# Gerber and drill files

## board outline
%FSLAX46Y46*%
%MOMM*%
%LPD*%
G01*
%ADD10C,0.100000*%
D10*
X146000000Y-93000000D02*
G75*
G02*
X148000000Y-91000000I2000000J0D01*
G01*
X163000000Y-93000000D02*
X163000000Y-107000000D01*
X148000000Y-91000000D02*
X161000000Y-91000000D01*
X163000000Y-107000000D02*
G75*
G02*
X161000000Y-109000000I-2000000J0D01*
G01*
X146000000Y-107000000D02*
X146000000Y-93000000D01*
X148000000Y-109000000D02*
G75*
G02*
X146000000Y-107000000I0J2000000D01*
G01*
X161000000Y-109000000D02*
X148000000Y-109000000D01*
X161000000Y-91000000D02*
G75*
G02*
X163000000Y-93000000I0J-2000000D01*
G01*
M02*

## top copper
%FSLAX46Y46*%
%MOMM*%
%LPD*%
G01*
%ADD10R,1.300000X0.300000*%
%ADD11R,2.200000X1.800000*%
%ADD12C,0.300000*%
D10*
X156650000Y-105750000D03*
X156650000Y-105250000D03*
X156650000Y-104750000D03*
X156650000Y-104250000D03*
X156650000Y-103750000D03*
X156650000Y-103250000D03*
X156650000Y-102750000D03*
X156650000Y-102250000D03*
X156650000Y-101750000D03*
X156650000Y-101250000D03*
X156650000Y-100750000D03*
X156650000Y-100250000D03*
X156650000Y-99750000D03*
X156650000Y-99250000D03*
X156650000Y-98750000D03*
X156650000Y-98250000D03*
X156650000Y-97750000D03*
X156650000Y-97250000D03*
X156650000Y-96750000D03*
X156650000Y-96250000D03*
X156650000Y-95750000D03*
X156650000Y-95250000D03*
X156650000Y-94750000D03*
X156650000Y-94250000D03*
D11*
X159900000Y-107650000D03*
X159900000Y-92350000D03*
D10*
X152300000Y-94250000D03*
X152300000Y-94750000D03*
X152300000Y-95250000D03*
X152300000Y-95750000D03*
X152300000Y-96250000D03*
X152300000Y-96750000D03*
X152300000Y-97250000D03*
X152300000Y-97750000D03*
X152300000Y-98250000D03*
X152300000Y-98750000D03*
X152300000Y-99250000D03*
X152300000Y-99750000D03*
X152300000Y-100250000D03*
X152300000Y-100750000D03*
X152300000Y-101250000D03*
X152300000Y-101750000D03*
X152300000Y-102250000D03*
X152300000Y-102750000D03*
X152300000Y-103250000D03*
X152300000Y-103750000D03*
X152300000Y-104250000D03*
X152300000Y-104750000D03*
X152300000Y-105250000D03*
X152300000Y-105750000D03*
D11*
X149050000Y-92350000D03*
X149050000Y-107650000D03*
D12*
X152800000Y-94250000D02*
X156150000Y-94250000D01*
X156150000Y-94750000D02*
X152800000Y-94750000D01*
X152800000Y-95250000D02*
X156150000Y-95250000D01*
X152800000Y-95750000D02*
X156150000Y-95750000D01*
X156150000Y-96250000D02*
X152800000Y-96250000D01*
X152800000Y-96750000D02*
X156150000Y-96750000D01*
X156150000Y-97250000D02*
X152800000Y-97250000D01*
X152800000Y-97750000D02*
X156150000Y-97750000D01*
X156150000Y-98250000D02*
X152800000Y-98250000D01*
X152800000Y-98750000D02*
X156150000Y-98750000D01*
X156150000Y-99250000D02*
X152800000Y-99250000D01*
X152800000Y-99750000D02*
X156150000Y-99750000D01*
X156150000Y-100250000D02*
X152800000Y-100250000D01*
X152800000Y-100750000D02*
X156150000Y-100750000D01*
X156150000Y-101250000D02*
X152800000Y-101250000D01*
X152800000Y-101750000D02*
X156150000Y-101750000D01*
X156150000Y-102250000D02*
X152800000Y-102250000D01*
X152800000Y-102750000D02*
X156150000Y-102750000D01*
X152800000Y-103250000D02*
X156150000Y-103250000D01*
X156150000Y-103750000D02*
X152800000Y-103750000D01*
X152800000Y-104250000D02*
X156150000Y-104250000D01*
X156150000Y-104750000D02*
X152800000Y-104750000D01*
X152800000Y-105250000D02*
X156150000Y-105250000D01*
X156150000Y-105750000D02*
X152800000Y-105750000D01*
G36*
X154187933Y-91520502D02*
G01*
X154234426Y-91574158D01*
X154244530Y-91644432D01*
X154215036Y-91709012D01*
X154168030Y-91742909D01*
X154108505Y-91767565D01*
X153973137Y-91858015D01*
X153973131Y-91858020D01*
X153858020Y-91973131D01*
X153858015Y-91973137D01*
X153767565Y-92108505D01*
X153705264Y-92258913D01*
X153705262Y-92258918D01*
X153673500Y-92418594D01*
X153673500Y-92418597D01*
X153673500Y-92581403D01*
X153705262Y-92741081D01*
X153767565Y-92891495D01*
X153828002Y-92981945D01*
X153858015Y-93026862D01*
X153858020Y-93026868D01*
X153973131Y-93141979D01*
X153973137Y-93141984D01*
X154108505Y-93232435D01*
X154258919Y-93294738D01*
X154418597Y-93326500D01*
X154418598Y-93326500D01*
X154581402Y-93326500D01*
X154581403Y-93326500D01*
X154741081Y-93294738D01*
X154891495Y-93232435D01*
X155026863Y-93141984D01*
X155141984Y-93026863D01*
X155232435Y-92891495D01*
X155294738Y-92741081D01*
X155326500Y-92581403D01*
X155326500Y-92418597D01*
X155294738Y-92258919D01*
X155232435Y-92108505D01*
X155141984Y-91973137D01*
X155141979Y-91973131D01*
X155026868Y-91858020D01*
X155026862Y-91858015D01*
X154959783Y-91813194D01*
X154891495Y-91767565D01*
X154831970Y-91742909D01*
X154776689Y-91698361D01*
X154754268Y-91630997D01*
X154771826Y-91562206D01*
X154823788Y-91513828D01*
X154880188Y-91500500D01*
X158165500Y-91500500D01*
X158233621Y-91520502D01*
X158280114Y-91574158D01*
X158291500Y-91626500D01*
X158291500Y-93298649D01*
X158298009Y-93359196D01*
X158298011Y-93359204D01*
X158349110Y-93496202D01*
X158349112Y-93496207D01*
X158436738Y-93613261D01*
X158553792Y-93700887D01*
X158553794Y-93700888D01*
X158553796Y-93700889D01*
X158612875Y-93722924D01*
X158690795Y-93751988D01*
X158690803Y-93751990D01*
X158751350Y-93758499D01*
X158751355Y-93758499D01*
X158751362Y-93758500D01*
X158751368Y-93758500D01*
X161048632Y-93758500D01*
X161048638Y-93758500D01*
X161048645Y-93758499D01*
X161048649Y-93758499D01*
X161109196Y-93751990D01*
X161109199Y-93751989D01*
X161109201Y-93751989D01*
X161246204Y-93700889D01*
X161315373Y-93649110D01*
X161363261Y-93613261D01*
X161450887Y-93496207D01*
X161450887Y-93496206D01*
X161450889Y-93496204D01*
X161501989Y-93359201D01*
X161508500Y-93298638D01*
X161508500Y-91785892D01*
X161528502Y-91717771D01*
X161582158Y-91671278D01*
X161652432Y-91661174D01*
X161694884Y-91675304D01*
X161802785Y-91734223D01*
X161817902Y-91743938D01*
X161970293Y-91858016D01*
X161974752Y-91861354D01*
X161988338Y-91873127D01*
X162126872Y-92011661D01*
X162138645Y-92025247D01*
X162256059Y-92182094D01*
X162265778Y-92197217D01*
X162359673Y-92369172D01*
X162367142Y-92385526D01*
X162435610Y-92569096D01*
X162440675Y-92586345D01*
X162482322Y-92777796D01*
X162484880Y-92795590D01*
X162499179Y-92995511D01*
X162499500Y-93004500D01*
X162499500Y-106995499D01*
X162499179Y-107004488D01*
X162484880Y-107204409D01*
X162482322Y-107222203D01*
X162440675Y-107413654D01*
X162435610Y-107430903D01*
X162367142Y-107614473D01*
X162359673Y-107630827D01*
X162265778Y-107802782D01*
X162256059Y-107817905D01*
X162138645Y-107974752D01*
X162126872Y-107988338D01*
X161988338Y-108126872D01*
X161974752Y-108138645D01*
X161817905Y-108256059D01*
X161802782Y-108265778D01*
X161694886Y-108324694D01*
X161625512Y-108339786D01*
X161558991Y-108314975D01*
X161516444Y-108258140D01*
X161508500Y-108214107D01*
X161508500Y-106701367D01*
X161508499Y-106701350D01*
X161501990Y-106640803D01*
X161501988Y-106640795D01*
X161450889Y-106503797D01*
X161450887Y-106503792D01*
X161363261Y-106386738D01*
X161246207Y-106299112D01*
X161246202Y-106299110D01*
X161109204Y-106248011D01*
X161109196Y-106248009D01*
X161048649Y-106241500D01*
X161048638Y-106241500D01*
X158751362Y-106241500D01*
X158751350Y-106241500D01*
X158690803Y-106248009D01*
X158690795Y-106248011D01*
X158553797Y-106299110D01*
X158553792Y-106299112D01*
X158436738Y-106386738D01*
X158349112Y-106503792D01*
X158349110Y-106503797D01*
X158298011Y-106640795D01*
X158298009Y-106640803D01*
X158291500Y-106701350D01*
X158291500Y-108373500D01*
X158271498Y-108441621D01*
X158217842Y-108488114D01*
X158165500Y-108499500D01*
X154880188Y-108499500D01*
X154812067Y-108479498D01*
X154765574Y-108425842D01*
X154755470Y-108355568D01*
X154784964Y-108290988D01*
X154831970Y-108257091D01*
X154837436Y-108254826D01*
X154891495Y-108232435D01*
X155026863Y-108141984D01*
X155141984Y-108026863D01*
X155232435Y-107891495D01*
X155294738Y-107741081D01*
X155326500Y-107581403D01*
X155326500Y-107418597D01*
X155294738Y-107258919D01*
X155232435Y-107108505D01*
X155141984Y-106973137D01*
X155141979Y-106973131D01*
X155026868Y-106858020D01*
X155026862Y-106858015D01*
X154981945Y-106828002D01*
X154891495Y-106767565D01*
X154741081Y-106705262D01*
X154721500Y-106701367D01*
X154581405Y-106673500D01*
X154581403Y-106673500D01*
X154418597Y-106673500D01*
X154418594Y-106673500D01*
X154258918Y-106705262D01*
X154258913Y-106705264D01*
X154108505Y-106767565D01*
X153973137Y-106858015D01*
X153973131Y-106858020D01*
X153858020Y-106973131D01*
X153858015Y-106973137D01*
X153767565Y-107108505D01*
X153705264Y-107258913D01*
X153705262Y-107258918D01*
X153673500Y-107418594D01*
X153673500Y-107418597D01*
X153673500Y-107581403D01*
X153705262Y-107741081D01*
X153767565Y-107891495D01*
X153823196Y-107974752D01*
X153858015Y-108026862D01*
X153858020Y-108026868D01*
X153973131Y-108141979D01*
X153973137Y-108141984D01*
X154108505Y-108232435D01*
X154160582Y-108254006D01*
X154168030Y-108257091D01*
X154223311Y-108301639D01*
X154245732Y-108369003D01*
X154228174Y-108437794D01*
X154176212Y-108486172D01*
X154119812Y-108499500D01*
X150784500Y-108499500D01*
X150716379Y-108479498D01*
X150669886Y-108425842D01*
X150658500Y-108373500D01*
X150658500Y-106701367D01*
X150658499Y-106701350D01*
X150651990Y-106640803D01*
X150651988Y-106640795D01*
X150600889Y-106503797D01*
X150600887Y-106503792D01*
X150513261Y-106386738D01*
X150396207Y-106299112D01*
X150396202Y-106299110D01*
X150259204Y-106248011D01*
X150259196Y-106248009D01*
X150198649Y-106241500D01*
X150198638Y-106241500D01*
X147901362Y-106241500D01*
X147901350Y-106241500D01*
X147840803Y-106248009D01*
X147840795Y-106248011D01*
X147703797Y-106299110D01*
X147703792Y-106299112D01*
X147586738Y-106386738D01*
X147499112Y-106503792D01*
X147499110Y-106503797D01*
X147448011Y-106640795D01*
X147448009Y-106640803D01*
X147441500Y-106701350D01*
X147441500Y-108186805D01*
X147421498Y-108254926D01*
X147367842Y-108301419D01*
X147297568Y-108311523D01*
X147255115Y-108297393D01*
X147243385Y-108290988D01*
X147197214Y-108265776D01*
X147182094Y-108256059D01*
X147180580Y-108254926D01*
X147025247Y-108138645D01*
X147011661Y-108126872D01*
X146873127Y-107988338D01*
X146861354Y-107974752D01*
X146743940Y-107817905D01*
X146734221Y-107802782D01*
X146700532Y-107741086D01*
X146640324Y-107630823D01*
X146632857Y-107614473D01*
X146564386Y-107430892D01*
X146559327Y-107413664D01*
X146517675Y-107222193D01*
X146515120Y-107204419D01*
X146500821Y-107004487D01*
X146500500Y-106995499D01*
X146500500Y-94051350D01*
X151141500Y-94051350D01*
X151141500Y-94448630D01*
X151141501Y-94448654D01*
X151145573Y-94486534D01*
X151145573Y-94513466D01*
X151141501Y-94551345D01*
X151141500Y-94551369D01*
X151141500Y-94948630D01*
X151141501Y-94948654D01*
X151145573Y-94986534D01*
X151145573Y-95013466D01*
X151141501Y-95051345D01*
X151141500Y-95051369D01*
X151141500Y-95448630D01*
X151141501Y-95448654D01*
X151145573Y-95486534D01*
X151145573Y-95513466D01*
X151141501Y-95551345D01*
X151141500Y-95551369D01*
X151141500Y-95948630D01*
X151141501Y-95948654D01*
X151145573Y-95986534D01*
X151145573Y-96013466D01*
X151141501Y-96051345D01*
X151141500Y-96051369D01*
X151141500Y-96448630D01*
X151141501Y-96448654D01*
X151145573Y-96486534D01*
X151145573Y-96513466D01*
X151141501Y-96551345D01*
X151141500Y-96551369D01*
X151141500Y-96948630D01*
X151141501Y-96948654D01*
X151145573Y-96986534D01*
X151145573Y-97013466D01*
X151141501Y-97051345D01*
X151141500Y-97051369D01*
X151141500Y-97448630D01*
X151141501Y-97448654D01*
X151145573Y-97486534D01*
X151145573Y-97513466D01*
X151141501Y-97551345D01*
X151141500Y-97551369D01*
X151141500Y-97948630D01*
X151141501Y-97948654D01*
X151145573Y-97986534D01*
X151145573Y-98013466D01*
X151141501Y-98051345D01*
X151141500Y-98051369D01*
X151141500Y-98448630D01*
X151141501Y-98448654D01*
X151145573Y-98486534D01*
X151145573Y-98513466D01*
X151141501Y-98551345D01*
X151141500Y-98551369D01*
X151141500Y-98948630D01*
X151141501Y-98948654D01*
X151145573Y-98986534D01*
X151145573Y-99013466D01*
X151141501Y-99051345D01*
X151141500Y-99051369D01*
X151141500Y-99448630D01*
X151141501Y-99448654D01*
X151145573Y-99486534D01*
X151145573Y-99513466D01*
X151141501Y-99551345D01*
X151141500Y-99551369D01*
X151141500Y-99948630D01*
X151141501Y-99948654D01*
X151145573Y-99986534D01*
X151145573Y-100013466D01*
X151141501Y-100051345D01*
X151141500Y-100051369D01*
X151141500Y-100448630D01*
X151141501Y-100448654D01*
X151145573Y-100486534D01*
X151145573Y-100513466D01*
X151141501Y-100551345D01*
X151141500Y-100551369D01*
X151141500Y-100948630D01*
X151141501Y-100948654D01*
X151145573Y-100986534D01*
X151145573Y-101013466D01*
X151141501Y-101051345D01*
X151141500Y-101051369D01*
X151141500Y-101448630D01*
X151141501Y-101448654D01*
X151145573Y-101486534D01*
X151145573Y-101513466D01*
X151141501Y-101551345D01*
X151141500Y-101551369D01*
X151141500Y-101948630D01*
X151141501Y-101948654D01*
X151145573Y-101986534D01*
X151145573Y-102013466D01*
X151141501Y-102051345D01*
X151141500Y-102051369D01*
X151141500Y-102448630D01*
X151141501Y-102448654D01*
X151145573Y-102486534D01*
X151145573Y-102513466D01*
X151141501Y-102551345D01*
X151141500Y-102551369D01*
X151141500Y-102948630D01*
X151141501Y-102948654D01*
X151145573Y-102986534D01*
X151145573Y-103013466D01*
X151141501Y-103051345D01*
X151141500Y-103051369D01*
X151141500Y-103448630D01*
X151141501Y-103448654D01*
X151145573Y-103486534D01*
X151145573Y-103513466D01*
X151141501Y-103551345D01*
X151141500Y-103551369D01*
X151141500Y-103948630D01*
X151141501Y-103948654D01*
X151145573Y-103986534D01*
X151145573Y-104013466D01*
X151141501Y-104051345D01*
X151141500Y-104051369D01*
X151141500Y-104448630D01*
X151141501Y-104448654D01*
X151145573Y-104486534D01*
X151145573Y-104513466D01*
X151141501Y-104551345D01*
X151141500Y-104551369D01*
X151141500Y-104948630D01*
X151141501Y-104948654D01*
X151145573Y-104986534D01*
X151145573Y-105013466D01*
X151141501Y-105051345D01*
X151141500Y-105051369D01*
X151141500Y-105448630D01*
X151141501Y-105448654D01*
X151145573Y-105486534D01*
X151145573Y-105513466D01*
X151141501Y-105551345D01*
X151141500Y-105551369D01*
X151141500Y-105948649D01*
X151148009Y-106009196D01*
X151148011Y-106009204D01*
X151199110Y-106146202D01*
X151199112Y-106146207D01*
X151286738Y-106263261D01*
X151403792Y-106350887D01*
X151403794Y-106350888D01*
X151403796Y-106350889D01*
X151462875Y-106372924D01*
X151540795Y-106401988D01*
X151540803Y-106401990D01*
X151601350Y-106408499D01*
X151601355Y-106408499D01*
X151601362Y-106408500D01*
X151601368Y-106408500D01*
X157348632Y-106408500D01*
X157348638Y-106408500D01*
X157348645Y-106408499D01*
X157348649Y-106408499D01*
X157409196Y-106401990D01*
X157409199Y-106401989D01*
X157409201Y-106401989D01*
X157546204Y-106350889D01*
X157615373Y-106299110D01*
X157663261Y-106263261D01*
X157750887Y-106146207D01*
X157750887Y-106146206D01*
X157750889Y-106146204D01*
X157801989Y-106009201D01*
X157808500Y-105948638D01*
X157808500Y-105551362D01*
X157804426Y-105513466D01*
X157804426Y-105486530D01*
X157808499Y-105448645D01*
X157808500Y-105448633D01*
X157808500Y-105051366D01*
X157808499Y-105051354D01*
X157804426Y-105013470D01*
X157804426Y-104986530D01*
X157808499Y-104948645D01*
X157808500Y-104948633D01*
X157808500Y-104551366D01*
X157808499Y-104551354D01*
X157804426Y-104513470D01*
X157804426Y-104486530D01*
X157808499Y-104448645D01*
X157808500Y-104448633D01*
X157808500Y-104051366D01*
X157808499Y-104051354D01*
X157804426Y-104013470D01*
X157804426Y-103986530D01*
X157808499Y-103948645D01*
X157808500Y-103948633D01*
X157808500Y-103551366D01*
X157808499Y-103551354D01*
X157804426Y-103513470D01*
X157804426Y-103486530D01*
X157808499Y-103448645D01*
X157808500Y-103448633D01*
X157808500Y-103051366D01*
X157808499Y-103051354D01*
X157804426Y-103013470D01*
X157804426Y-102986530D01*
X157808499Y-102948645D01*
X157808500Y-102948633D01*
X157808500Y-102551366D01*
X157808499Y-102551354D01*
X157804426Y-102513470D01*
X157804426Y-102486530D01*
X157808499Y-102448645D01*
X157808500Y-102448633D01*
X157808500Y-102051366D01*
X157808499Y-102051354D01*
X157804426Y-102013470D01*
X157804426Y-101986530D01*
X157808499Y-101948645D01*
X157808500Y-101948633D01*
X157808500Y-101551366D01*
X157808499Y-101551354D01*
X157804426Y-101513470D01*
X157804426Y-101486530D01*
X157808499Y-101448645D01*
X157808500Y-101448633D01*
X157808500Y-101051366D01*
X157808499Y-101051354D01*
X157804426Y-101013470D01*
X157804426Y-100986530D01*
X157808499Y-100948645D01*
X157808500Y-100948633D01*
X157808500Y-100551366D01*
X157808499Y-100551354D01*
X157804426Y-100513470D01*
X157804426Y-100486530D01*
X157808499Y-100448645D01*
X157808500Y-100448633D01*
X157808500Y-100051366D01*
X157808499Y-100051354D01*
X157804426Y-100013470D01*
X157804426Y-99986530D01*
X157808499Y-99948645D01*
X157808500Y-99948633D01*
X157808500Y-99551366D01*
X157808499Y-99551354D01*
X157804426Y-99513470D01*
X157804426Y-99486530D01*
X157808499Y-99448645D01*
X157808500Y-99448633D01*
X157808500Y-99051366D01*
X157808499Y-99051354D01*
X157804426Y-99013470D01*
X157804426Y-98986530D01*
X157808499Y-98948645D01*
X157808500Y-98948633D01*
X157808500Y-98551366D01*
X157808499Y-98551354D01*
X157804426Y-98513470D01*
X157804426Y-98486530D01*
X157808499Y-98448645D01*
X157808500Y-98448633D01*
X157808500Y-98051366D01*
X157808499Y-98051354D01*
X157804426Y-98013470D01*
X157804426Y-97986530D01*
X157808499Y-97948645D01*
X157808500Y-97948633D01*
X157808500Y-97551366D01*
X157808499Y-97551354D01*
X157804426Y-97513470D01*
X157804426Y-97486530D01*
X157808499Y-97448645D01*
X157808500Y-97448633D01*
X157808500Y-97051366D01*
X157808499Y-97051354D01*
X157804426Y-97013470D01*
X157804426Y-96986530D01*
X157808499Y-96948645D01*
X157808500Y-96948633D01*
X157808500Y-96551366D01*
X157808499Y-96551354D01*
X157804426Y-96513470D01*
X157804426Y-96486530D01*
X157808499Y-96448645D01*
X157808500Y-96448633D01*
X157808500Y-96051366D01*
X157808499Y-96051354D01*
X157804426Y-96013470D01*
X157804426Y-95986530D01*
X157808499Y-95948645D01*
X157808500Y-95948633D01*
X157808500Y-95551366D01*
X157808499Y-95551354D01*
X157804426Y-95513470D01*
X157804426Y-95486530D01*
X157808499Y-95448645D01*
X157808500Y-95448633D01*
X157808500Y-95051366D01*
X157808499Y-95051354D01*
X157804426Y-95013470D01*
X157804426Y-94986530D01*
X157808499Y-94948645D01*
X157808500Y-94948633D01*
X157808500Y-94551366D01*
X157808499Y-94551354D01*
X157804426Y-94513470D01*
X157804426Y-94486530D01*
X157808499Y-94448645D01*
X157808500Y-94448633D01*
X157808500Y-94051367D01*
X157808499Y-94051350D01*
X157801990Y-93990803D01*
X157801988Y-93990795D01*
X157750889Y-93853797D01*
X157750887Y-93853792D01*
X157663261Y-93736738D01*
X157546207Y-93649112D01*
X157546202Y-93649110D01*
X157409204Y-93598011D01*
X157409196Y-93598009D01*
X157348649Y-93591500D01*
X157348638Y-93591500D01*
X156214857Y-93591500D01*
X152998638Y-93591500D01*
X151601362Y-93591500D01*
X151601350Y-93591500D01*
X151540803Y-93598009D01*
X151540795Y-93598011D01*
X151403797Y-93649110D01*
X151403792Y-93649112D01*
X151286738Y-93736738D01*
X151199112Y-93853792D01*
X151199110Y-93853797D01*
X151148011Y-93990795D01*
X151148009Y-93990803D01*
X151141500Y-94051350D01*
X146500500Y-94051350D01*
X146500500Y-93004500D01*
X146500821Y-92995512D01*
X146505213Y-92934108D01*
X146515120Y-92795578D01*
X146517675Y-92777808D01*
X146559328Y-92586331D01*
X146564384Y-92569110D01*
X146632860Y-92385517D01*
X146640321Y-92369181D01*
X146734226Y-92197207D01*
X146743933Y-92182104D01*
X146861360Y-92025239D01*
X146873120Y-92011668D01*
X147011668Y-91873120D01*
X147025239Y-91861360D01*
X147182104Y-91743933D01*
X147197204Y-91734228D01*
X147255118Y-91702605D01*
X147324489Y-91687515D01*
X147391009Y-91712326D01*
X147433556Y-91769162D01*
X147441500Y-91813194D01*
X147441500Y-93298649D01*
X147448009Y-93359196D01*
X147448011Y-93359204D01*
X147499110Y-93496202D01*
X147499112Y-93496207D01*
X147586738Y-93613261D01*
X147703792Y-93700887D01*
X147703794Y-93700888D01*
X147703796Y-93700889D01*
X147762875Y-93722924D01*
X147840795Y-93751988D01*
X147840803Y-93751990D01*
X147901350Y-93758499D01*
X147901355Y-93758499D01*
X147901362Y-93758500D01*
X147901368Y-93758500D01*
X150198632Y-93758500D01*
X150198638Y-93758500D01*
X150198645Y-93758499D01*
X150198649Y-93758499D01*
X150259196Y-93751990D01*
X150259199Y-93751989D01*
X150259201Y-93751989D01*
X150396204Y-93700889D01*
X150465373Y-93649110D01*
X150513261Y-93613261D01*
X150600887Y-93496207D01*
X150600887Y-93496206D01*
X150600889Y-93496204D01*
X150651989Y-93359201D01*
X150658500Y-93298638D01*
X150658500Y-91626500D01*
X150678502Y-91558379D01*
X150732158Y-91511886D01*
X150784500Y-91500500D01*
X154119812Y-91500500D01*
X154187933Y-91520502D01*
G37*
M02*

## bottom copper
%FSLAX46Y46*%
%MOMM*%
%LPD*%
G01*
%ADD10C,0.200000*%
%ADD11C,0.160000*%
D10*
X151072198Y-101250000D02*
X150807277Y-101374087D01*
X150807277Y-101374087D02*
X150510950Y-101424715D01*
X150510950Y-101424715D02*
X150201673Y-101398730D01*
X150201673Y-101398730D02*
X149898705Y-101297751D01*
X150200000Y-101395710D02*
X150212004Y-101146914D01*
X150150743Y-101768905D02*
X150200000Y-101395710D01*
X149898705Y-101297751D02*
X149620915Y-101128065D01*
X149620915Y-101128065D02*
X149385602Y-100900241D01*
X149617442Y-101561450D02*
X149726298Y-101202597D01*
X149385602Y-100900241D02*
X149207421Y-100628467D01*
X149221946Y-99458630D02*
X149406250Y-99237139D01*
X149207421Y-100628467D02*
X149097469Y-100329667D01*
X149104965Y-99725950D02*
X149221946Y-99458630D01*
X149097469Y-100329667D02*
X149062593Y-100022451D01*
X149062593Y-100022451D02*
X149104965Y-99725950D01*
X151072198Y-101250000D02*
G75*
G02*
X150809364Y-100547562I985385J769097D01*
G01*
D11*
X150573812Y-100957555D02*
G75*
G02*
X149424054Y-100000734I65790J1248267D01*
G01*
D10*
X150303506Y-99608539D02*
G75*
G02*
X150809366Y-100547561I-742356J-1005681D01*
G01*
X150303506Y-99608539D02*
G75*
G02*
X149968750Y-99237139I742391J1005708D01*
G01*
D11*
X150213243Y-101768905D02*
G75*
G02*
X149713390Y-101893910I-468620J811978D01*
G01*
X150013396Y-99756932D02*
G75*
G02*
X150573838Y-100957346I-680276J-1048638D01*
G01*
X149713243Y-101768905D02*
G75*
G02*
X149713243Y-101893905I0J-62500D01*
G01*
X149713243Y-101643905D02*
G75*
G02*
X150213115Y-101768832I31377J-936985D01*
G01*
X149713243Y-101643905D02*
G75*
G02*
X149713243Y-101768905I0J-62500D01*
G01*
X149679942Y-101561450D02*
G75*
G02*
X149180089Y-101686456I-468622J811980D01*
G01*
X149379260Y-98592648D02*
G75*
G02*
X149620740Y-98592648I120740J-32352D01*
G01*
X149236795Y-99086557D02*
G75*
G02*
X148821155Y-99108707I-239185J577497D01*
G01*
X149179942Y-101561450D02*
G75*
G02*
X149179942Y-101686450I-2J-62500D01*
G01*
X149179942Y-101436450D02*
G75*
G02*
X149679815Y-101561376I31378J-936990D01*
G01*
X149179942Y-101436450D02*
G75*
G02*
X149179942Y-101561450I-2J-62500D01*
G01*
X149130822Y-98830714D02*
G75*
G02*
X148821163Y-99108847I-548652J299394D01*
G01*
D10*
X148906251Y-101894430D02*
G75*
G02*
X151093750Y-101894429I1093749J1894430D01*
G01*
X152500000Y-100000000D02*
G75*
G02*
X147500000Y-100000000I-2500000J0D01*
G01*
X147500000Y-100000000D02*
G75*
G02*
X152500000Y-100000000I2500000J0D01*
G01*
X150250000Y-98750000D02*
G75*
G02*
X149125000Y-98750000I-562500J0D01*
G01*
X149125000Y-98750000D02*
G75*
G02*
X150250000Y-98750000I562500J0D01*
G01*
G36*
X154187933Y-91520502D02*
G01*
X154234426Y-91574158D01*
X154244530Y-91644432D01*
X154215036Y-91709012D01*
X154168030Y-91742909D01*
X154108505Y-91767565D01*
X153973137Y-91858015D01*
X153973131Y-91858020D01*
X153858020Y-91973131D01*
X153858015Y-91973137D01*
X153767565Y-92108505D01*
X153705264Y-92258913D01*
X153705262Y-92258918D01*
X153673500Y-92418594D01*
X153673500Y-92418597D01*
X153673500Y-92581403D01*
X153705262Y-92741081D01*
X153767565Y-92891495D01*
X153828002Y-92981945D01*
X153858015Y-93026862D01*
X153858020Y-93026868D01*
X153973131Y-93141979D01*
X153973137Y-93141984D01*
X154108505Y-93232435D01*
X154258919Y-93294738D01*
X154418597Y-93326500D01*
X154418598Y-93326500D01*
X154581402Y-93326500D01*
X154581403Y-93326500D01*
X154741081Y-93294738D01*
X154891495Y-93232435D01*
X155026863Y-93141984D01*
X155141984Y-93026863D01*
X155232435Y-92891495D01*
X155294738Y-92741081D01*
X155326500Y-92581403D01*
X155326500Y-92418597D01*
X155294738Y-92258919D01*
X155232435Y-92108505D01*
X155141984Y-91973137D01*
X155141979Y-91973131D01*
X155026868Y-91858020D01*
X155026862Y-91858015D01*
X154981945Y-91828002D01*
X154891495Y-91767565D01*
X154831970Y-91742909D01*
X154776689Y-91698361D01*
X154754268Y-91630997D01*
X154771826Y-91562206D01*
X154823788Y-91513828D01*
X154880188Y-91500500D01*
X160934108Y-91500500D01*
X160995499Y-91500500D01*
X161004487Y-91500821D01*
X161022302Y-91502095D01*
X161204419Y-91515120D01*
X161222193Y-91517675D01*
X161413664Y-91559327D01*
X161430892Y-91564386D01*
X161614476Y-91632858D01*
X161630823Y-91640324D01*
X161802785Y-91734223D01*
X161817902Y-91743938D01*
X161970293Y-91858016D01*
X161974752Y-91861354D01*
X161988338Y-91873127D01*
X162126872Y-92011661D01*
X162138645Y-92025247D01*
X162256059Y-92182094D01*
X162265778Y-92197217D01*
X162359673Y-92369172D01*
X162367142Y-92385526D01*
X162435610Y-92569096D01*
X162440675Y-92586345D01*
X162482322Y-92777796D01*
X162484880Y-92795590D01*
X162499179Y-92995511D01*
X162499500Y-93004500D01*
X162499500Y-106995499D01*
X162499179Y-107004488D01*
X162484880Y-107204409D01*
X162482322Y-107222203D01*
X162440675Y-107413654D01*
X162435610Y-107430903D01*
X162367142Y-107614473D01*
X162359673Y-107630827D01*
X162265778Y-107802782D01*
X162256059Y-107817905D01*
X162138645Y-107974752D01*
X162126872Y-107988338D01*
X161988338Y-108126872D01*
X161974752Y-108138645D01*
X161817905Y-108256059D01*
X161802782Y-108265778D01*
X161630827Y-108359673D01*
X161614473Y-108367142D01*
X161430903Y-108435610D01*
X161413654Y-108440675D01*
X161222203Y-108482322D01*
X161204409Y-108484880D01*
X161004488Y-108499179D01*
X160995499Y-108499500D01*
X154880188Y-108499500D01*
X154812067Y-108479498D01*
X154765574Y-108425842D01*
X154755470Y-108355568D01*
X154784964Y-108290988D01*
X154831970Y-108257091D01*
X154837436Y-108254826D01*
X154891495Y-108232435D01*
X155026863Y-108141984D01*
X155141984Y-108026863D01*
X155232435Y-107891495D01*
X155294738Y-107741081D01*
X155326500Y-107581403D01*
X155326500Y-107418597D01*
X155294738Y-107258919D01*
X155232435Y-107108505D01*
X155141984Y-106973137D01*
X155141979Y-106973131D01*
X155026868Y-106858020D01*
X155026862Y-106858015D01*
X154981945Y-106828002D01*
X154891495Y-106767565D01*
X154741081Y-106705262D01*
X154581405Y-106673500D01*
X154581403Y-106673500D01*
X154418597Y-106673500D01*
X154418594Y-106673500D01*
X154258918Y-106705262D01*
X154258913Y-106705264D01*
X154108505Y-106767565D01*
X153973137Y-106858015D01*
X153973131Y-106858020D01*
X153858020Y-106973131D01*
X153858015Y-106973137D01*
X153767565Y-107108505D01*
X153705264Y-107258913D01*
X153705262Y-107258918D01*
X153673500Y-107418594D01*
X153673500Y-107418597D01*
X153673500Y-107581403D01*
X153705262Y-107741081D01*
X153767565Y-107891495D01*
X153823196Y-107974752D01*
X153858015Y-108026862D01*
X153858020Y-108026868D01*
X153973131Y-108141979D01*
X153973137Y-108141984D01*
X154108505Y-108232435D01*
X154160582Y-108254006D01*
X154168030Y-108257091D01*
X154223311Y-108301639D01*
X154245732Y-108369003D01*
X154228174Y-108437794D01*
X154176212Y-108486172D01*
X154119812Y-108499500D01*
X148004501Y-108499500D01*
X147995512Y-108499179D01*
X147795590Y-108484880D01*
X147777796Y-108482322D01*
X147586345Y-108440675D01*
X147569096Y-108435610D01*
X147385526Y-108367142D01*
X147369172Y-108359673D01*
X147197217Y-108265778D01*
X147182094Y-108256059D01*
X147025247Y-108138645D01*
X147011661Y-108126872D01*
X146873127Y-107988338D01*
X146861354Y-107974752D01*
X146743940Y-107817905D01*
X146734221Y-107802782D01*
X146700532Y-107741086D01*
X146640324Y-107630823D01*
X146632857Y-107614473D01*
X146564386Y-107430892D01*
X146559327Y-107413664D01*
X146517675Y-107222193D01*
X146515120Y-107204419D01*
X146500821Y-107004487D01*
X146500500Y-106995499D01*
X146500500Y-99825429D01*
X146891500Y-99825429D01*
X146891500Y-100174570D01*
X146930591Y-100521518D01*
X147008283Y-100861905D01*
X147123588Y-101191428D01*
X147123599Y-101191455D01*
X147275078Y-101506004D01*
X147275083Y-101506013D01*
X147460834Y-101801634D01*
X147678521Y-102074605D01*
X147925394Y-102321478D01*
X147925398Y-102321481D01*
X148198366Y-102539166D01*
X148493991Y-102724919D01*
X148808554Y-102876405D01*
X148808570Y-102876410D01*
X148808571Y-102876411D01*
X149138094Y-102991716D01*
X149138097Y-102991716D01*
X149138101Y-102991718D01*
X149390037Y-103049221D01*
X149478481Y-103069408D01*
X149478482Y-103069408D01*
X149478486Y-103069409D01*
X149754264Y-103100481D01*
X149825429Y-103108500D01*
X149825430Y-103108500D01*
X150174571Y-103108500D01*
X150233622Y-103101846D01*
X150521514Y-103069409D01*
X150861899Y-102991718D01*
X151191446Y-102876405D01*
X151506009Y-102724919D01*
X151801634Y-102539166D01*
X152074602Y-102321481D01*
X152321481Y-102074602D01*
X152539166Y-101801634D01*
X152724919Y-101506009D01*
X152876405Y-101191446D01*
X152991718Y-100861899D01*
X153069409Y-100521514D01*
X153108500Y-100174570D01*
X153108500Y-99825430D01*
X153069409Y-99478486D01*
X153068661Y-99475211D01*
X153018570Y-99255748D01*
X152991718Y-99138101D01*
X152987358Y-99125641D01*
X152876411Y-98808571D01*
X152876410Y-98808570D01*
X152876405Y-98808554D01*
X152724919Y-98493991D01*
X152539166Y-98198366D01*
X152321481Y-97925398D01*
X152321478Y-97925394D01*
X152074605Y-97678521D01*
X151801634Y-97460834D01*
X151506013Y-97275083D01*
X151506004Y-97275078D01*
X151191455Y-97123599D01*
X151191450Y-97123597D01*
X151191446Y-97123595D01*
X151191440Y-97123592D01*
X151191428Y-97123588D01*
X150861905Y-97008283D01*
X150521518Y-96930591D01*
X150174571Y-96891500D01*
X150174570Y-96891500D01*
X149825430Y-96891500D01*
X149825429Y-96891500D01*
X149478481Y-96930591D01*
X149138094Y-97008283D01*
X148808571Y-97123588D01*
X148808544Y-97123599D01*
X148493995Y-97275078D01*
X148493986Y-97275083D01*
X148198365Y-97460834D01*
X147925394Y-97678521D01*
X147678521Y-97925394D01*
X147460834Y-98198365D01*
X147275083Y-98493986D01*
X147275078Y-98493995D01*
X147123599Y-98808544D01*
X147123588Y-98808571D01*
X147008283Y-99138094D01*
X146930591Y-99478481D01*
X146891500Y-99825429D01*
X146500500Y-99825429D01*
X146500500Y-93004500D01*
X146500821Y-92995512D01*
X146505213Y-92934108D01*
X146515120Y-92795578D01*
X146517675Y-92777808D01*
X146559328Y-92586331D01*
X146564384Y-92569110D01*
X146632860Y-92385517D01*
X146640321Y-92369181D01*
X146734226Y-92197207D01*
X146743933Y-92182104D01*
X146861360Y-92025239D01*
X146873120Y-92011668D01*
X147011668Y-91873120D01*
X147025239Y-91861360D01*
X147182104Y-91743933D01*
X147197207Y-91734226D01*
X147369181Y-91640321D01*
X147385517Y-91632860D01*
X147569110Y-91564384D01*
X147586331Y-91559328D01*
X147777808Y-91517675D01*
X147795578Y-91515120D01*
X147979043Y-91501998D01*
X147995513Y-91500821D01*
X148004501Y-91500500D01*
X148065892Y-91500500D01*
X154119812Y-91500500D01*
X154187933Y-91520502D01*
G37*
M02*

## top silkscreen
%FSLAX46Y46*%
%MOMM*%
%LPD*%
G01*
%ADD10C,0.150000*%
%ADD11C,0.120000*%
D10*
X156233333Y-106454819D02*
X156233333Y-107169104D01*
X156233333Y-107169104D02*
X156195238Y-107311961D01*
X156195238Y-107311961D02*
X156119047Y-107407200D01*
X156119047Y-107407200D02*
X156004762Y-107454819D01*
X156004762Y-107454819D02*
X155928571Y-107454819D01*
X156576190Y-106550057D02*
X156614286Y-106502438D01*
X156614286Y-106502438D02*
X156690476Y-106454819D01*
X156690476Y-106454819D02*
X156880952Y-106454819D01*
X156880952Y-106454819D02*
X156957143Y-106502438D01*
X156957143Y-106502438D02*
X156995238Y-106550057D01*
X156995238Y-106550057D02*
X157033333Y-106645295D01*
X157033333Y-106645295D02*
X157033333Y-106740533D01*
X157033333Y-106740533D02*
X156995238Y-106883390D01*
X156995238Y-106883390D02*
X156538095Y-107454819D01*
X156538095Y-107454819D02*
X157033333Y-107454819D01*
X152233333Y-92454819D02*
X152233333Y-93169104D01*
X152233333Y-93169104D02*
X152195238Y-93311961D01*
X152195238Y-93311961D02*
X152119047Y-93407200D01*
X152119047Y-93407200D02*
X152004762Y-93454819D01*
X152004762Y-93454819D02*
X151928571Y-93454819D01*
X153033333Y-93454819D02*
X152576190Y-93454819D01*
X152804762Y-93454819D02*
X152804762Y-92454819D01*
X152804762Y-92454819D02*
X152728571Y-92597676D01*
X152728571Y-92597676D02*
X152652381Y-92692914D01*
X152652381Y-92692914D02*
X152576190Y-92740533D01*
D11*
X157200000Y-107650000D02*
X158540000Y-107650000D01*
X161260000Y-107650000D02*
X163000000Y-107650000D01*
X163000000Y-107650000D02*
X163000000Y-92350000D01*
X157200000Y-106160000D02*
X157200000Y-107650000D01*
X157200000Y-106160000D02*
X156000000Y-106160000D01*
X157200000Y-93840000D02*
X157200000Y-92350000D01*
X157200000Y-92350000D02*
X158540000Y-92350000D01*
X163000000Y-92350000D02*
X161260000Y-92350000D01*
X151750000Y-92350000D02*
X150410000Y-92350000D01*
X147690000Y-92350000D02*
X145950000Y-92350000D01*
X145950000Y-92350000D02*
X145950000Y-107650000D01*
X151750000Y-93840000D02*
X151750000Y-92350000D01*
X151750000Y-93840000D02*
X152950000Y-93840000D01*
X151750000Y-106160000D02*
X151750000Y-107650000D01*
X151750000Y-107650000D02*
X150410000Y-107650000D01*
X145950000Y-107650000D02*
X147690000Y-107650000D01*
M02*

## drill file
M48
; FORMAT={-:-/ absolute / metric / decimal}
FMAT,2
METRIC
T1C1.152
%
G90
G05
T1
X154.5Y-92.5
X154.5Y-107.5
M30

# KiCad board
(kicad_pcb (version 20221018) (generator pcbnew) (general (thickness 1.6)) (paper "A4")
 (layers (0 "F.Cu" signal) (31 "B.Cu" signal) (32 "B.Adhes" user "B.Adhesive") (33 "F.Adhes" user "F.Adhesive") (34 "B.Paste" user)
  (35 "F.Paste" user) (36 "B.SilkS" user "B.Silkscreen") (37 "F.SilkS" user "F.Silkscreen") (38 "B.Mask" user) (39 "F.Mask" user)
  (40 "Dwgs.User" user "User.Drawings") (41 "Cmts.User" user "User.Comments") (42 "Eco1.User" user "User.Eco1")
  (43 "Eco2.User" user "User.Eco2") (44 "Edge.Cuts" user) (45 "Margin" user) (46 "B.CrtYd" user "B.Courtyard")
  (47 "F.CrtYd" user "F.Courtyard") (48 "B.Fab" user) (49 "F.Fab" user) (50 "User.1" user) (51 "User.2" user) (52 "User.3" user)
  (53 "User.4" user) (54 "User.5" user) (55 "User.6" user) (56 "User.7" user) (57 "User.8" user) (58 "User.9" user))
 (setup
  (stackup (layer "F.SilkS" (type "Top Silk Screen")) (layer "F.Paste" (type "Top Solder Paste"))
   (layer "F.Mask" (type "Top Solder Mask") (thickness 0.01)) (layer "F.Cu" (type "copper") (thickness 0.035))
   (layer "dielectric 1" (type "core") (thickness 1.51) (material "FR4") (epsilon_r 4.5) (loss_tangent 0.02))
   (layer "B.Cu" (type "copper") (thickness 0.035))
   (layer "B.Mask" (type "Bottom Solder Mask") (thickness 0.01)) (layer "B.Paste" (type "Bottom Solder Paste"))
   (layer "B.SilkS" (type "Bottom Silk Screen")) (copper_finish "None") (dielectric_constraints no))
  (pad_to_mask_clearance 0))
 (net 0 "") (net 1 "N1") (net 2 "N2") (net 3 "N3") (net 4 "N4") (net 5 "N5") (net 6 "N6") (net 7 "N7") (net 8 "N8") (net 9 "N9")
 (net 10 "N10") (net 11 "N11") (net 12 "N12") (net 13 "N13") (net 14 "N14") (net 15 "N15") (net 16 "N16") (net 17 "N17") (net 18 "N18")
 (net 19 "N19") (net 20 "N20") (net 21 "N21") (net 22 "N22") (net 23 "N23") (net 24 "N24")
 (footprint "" (layer "F.Cu") (at 154.5 92.5)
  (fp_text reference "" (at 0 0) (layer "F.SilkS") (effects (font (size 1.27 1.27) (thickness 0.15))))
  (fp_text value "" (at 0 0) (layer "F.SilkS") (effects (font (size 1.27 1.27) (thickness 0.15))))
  (pad "" np_thru_hole circle (at 0 0) (size 1.152 1.152) (drill 1.152) (layers "F&B.Cu" "*.Mask")))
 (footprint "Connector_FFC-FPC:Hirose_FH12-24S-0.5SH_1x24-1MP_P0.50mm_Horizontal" (layer "F.Cu") (at 158.5 100 90)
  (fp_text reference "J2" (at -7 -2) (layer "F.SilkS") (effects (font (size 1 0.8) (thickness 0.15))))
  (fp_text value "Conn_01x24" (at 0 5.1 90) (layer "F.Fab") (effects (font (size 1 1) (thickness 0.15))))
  (fp_line (start -7.65 -1.3) (end -7.65 0.04) (stroke (width 0.12) (type solid)) (layer "F.SilkS"))
  (fp_line (start -7.65 2.76) (end -7.65 4.5) (stroke (width 0.12) (type solid)) (layer "F.SilkS"))
  (fp_line (start -7.65 4.5) (end 7.65 4.5) (stroke (width 0.12) (type solid)) (layer "F.SilkS"))
  (fp_line (start -6.16 -1.3) (end -7.65 -1.3) (stroke (width 0.12) (type solid)) (layer "F.SilkS"))
  (fp_line (start -6.16 -1.3) (end -6.16 -2.5) (stroke (width 0.12) (type solid)) (layer "F.SilkS"))
  (fp_line (start 6.16 -1.3) (end 7.65 -1.3) (stroke (width 0.12) (type solid)) (layer "F.SilkS"))
  (fp_line (start 7.65 -1.3) (end 7.65 0.04) (stroke (width 0.12) (type solid)) (layer "F.SilkS"))
  (fp_line (start 7.65 4.5) (end 7.65 2.76) (stroke (width 0.12) (type solid)) (layer "F.SilkS"))
  (pad "1" smd rect (at -5.75 -1.85 90) (size 0.3 1.3) (layers "F.Cu" "F.Paste" "F.Mask") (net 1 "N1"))
  (pad "2" smd rect (at -5.25 -1.85 90) (size 0.3 1.3) (layers "F.Cu" "F.Paste" "F.Mask") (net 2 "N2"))
  (pad "3" smd rect (at -4.75 -1.85 90) (size 0.3 1.3) (layers "F.Cu" "F.Paste" "F.Mask") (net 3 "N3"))
  (pad "4" smd rect (at -4.25 -1.85 90) (size 0.3 1.3) (layers "F.Cu" "F.Paste" "F.Mask") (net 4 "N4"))
  (pad "5" smd rect (at -3.75 -1.85 90) (size 0.3 1.3) (layers "F.Cu" "F.Paste" "F.Mask") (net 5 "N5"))
  (pad "6" smd rect (at -3.25 -1.85 90) (size 0.3 1.3) (layers "F.Cu" "F.Paste" "F.Mask") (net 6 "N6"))
  (pad "7" smd rect (at -2.75 -1.85 90) (size 0.3 1.3) (layers "F.Cu" "F.Paste" "F.Mask") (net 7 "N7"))
  (pad "8" smd rect (at -2.25 -1.85 90) (size 0.3 1.3) (layers "F.Cu" "F.Paste" "F.Mask") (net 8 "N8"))
  (pad "9" smd rect (at -1.75 -1.85 90) (size 0.3 1.3) (layers "F.Cu" "F.Paste" "F.Mask") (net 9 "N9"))
  (pad "10" smd rect (at -1.25 -1.85 90) (size 0.3 1.3) (layers "F.Cu" "F.Paste" "F.Mask") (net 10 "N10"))
  (pad "11" smd rect (at -0.75 -1.85 90) (size 0.3 1.3) (layers "F.Cu" "F.Paste" "F.Mask") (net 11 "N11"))
  (pad "12" smd rect (at -0.25 -1.85 90) (size 0.3 1.3) (layers "F.Cu" "F.Paste" "F.Mask") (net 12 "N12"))
  (pad "13" smd rect (at 0.25 -1.85 90) (size 0.3 1.3) (layers "F.Cu" "F.Paste" "F.Mask") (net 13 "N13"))
  (pad "14" smd rect (at 0.75 -1.85 90) (size 0.3 1.3) (layers "F.Cu" "F.Paste" "F.Mask") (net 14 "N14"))
  (pad "15" smd rect (at 1.25 -1.85 90) (size 0.3 1.3) (layers "F.Cu" "F.Paste" "F.Mask") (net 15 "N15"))
  (pad "16" smd rect (at 1.75 -1.85 90) (size 0.3 1.3) (layers "F.Cu" "F.Paste" "F.Mask") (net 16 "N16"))
  (pad "17" smd rect (at 2.25 -1.85 90) (size 0.3 1.3) (layers "F.Cu" "F.Paste" "F.Mask") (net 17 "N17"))
  (pad "18" smd rect (at 2.75 -1.85 90) (size 0.3 1.3) (layers "F.Cu" "F.Paste" "F.Mask") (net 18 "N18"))
  (pad "19" smd rect (at 3.25 -1.85 90) (size 0.3 1.3) (layers "F.Cu" "F.Paste" "F.Mask") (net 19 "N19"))
  (pad "20" smd rect (at 3.75 -1.85 90) (size 0.3 1.3) (layers "F.Cu" "F.Paste" "F.Mask") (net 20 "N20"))
  (pad "21" smd rect (at 4.25 -1.85 90) (size 0.3 1.3) (layers "F.Cu" "F.Paste" "F.Mask") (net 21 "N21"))
  (pad "22" smd rect (at 4.75 -1.85 90) (size 0.3 1.3) (layers "F.Cu" "F.Paste" "F.Mask") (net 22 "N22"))
  (pad "23" smd rect (at 5.25 -1.85 90) (size 0.3 1.3) (layers "F.Cu" "F.Paste" "F.Mask") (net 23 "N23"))
  (pad "24" smd rect (at 5.75 -1.85 90) (size 0.3 1.3) (layers "F.Cu" "F.Paste" "F.Mask") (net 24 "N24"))
  (pad "MP" smd rect (at -7.65 1.4 90) (size 1.8 2.2) (layers "F.Cu" "F.Paste" "F.Mask"))
  (pad "MP" smd rect (at 7.65 1.4 90) (size 1.8 2.2) (layers "F.Cu" "F.Paste" "F.Mask")))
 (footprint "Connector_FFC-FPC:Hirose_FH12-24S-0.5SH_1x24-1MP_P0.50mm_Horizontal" (layer "F.Cu") (at 150.45 100 -90)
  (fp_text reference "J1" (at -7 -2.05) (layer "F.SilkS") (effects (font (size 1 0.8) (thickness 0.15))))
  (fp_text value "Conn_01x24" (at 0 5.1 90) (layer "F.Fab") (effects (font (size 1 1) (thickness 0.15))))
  (fp_line (start -7.65 -1.3) (end -7.65 0.04) (stroke (width 0.12) (type solid)) (layer "F.SilkS"))
  (fp_line (start -7.65 2.76) (end -7.65 4.5) (stroke (width 0.12) (type solid)) (layer "F.SilkS"))
  (fp_line (start -7.65 4.5) (end 7.65 4.5) (stroke (width 0.12) (type solid)) (layer "F.SilkS"))
  (fp_line (start -6.16 -1.3) (end -7.65 -1.3) (stroke (width 0.12) (type solid)) (layer "F.SilkS"))
  (fp_line (start -6.16 -1.3) (end -6.16 -2.5) (stroke (width 0.12) (type solid)) (layer "F.SilkS"))
  (fp_line (start 6.16 -1.3) (end 7.65 -1.3) (stroke (width 0.12) (type solid)) (layer "F.SilkS"))
  (fp_line (start 7.65 -1.3) (end 7.65 0.04) (stroke (width 0.12) (type solid)) (layer "F.SilkS"))
  (fp_line (start 7.65 4.5) (end 7.65 2.76) (stroke (width 0.12) (type solid)) (layer "F.SilkS"))
  (pad "1" smd rect (at -5.75 -1.85 270) (size 0.3 1.3) (layers "F.Cu" "F.Paste" "F.Mask") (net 24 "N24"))
  (pad "2" smd rect (at -5.25 -1.85 270) (size 0.3 1.3) (layers "F.Cu" "F.Paste" "F.Mask") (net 23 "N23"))
  (pad "3" smd rect (at -4.75 -1.85 270) (size 0.3 1.3) (layers "F.Cu" "F.Paste" "F.Mask") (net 22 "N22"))
  (pad "4" smd rect (at -4.25 -1.85 270) (size 0.3 1.3) (layers "F.Cu" "F.Paste" "F.Mask") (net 21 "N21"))
  (pad "5" smd rect (at -3.75 -1.85 270) (size 0.3 1.3) (layers "F.Cu" "F.Paste" "F.Mask") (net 20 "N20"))
  (pad "6" smd rect (at -3.25 -1.85 270) (size 0.3 1.3) (layers "F.Cu" "F.Paste" "F.Mask") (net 19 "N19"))
  (pad "7" smd rect (at -2.75 -1.85 270) (size 0.3 1.3) (layers "F.Cu" "F.Paste" "F.Mask") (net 18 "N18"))
  (pad "8" smd rect (at -2.25 -1.85 270) (size 0.3 1.3) (layers "F.Cu" "F.Paste" "F.Mask") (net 17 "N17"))
  (pad "9" smd rect (at -1.75 -1.85 270) (size 0.3 1.3) (layers "F.Cu" "F.Paste" "F.Mask") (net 16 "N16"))
  (pad "10" smd rect (at -1.25 -1.85 270) (size 0.3 1.3) (layers "F.Cu" "F.Paste" "F.Mask") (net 15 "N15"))
  (pad "11" smd rect (at -0.75 -1.85 270) (size 0.3 1.3) (layers "F.Cu" "F.Paste" "F.Mask") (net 14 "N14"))
  (pad "12" smd rect (at -0.25 -1.85 270) (size 0.3 1.3) (layers "F.Cu" "F.Paste" "F.Mask") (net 13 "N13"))
  (pad "13" smd rect (at 0.25 -1.85 270) (size 0.3 1.3) (layers "F.Cu" "F.Paste" "F.Mask") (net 12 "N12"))
  (pad "14" smd rect (at 0.75 -1.85 270) (size 0.3 1.3) (layers "F.Cu" "F.Paste" "F.Mask") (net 11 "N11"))
  (pad "15" smd rect (at 1.25 -1.85 270) (size 0.3 1.3) (layers "F.Cu" "F.Paste" "F.Mask") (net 10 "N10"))
  (pad "16" smd rect (at 1.75 -1.85 270) (size 0.3 1.3) (layers "F.Cu" "F.Paste" "F.Mask") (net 9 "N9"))
  (pad "17" smd rect (at 2.25 -1.85 270) (size 0.3 1.3) (layers "F.Cu" "F.Paste" "F.Mask") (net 8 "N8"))
  (pad "18" smd rect (at 2.75 -1.85 270) (size 0.3 1.3) (layers "F.Cu" "F.Paste" "F.Mask") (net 7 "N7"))
  (pad "19" smd rect (at 3.25 -1.85 270) (size 0.3 1.3) (layers "F.Cu" "F.Paste" "F.Mask") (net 6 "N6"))
  (pad "20" smd rect (at 3.75 -1.85 270) (size 0.3 1.3) (layers "F.Cu" "F.Paste" "F.Mask") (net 5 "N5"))
  (pad "21" smd rect (at 4.25 -1.85 270) (size 0.3 1.3) (layers "F.Cu" "F.Paste" "F.Mask") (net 4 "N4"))
  (pad "22" smd rect (at 4.75 -1.85 270) (size 0.3 1.3) (layers "F.Cu" "F.Paste" "F.Mask") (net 3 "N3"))
  (pad "23" smd rect (at 5.25 -1.85 270) (size 0.3 1.3) (layers "F.Cu" "F.Paste" "F.Mask") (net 2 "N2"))
  (pad "24" smd rect (at 5.75 -1.85 270) (size 0.3 1.3) (layers "F.Cu" "F.Paste" "F.Mask") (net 1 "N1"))
  (pad "MP" smd rect (at -7.65 1.4 270) (size 1.8 2.2) (layers "F.Cu" "F.Paste" "F.Mask"))
  (pad "MP" smd rect (at 7.65 1.4 270) (size 1.8 2.2) (layers "F.Cu" "F.Paste" "F.Mask")))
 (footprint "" (layer "F.Cu") (at 154.5 107.5)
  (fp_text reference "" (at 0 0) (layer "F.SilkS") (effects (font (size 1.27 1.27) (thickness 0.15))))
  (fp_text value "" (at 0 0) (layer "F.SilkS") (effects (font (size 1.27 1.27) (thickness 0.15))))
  (pad "" np_thru_hole circle (at 0 0) (size 1.152 1.152) (drill 1.152) (layers "F&B.Cu" "*.Mask")))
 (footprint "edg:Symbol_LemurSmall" (layer "B.Cu") (at 160 100 180)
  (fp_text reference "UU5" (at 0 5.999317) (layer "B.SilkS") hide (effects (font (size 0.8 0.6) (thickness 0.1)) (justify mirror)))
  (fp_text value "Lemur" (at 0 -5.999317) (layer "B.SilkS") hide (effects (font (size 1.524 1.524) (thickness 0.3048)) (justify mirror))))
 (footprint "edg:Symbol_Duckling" (layer "B.Cu") (at 150 100 180)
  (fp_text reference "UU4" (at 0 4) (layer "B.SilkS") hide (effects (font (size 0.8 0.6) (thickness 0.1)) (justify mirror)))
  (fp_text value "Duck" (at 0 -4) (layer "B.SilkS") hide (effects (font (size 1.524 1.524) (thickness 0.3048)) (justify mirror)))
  (fp_line (start -1.072198 -1.25) (end -0.807277 -1.374087) (stroke (width 0.2) (type solid)) (layer "B.Cu"))
  (fp_line (start -0.807277 -1.374087) (end -0.51095 -1.424715) (stroke (width 0.2) (type solid)) (layer "B.Cu"))
  (fp_line (start -0.51095 -1.424715) (end -0.201673 -1.39873) (stroke (width 0.2) (type solid)) (layer "B.Cu"))
  (fp_line (start -0.201673 -1.39873) (end 0.101295 -1.297751) (stroke (width 0.2) (type solid)) (layer "B.Cu"))
  (fp_line (start -0.2 -1.39571) (end -0.212004 -1.146914) (stroke (width 0.2) (type solid)) (layer "B.Cu"))
  (fp_line (start -0.150743 -1.768905) (end -0.2 -1.39571) (stroke (width 0.2) (type solid)) (layer "B.Cu"))
  (fp_line (start 0.101295 -1.297751) (end 0.379085 -1.128065) (stroke (width 0.2) (type solid)) (layer "B.Cu"))
  (fp_line (start 0.379085 -1.128065) (end 0.614398 -0.900241) (stroke (width 0.2) (type solid)) (layer "B.Cu"))
  (fp_line (start 0.382558 -1.56145) (end 0.273702 -1.202597) (stroke (width 0.2) (type solid)) (layer "B.Cu"))
  (fp_line (start 0.614398 -0.900241) (end 0.792579 -0.628467) (stroke (width 0.2) (type solid)) (layer "B.Cu"))
  (fp_line (start 0.778054 0.54137) (end 0.59375 0.762861) (stroke (width 0.2) (type solid)) (layer "B.Cu"))
  (fp_line (start 0.792579 -0.628467) (end 0.902531 -0.329667) (stroke (width 0.2) (type solid)) (layer "B.Cu"))
  (fp_line (start 0.895035 0.27405) (end 0.778054 0.54137) (stroke (width 0.2) (type solid)) (layer "B.Cu"))
  (fp_line (start 0.902531 -0.329667) (end 0.937407 -0.022451) (stroke (width 0.2) (type solid)) (layer "B.Cu"))
  (fp_line (start 0.937407 -0.022451) (end 0.895035 0.27405) (stroke (width 0.2) (type solid)) (layer "B.Cu"))
  (fp_arc (start -1.072198 -1.25) (mid -0.886856 -0.918958) (end -0.809364 -0.547562) (stroke (width 0.2) (type solid)) (layer "B.Cu"))
  (fp_arc (start -0.573812 -0.957555) (mid 0.159981 -0.670103) (end 0.575946 -0.000734) (stroke (width 0.16) (type solid)) (layer "B.Cu"))
  (fp_arc (start -0.303506 0.391461) (mid -0.66162 -0.021386) (end -0.809366 -0.547561) (stroke (width 0.2) (type solid)) (layer "B.Cu"))
  (fp_arc (start -0.303506 0.391461) (mid -0.117369 0.560253) (end 0.03125 0.762861) (stroke (width 0.2) (type solid)) (layer "B.Cu"))
  (fp_arc (start -0.213243 -1.768905) (mid 0.027927 -1.866421) (end 0.28661 -1.89391) (stroke (width 0.16) (type solid)) (layer "B.Cu"))
  (fp_arc (start -0.013396 0.243068) (mid -0.465729 -0.276784) (end -0.573838 -0.957346) (stroke (width 0.16) (type solid)) (layer "B.Cu"))
  (fp_arc (start 0.286757 -1.768905) (mid 0.224257 -1.831405) (end 0.286757 -1.893905) (stroke (width 0.16) (type solid)) (layer "B.Cu"))
  (fp_arc (start 0.286757 -1.643905) (mid 0.02807 -1.671354) (end -0.213115 -1.768832) (stroke (width 0.16) (type solid)) (layer "B.Cu"))
  (fp_arc (start 0.286757 -1.643905) (mid 0.224257 -1.706405) (end 0.286757 -1.768905) (stroke (width 0.16) (type solid)) (layer "B.Cu"))
  (fp_arc (start 0.320058 -1.56145) (mid 0.561228 -1.658966) (end 0.819911 -1.686455) (stroke (width 0.16) (type solid)) (layer "B.Cu"))
  (fp_arc (start 0.62074 1.407352) (mid 0.5 1.499999) (end 0.37926 1.407352) (stroke (width 0.16) (type solid)) (layer "B.Cu"))
  (fp_arc (start 0.763205 0.913443) (mid 0.969128 0.866757) (end 1.178844 0.891296) (stroke (width 0.16) (type solid)) (layer "B.Cu"))
  (fp_arc (start 0.820058 -1.56145) (mid 0.75756 -1.62395) (end 0.820058 -1.68645) (stroke (width 0.16) (type solid)) (layer "B.Cu"))
  (fp_arc (start 0.820058 -1.43645) (mid 0.561371 -1.463899) (end 0.320186 -1.561377) (stroke (width 0.16) (type solid)) (layer "B.Cu"))
  (fp_arc (start 0.820058 -1.43645) (mid 0.75756 -1.49895) (end 0.820058 -1.56145) (stroke (width 0.16) (type solid)) (layer "B.Cu"))
  (fp_arc (start 0.869178 1.169286) (mid 1.000175 1.003684) (end 1.178836 0.891151) (stroke (width 0.16) (type solid)) (layer "B.Cu"))
  (fp_arc (start 1.093749 -1.89443) (mid 0.000001 2.187499) (end -1.09375 -1.894429) (stroke (width 0.2) (type solid)) (layer "B.Cu"))
  (fp_circle (center 0 0) (end 2.5 0) (stroke (width 0.2) (type solid)) (fill none) (layer "B.Cu"))
  (fp_circle (center 0.3125 1.25) (end 0.875 1.25) (stroke (width 0.2) (type solid)) (fill none) (layer "B.Cu")))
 (gr_arc (start 146 93) (mid 146.585786 91.585786) (end 148 91) (stroke (width 0.1) (type solid)) (layer "Edge.Cuts"))
 (gr_line (start 163 93) (end 163 107) (stroke (width 0.1) (type solid)) (layer "Edge.Cuts"))
 (gr_line (start 148 91) (end 161 91) (stroke (width 0.1) (type solid)) (layer "Edge.Cuts"))
 (gr_arc (start 163 107) (mid 162.414214 108.414214) (end 161 109) (stroke (width 0.1) (type solid)) (layer "Edge.Cuts"))
 (gr_line (start 146 107) (end 146 93) (stroke (width 0.1) (type solid)) (layer "Edge.Cuts"))
 (gr_arc (start 148 109) (mid 146.585786 108.414214) (end 146 107) (stroke (width 0.1) (type solid)) (layer "Edge.Cuts"))
 (gr_line (start 161 109) (end 148 109) (stroke (width 0.1) (type solid)) (layer "Edge.Cuts"))
 (gr_arc (start 161 91) (mid 162.414214 91.585786) (end 163 93) (stroke (width 0.1) (type solid)) (layer "Edge.Cuts"))
 (segment (start 152.8 94.25) (end 156.15 94.25) (width 0.3) (layer "F.Cu") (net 24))
 (segment (start 156.15 94.75) (end 152.8 94.75) (width 0.3) (layer "F.Cu") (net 23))
 (segment (start 152.8 95.25) (end 156.15 95.25) (width 0.3) (layer "F.Cu") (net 22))
 (segment (start 152.8 95.75) (end 156.15 95.75) (width 0.3) (layer "F.Cu") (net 21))
 (segment (start 156.15 96.25) (end 152.8 96.25) (width 0.3) (layer "F.Cu") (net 20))
 (segment (start 152.8 96.75) (end 156.15 96.75) (width 0.3) (layer "F.Cu") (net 19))
 (segment (start 156.15 97.25) (end 152.8 97.25) (width 0.3) (layer "F.Cu") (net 18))
 (segment (start 152.8 97.75) (end 156.15 97.75) (width 0.3) (layer "F.Cu") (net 17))
 (segment (start 156.15 98.25) (end 152.8 98.25) (width 0.3) (layer "F.Cu") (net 16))
 (segment (start 152.8 98.75) (end 156.15 98.75) (width 0.3) (layer "F.Cu") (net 15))
 (segment (start 156.15 99.25) (end 152.8 99.25) (width 0.3) (layer "F.Cu") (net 14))
 (segment (start 152.8 99.75) (end 156.15 99.75) (width 0.3) (layer "F.Cu") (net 13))
 (segment (start 156.15 100.25) (end 152.8 100.25) (width 0.3) (layer "F.Cu") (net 12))
 (segment (start 152.8 100.75) (end 156.15 100.75) (width 0.3) (layer "F.Cu") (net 11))
 (segment (start 156.15 101.25) (end 152.8 101.25) (width 0.3) (layer "F.Cu") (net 10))
 (segment (start 152.8 101.75) (end 156.15 101.75) (width 0.3) (layer "F.Cu") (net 9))
 (segment (start 156.15 102.25) (end 152.8 102.25) (width 0.3) (layer "F.Cu") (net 8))
 (segment (start 152.8 102.75) (end 156.15 102.75) (width 0.3) (layer "F.Cu") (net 7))
 (segment (start 152.8 103.25) (end 156.15 103.25) (width 0.3) (layer "F.Cu") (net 6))
 (segment (start 156.15 103.75) (end 152.8 103.75) (width 0.3) (layer "F.Cu") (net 5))
 (segment (start 152.8 104.25) (end 156.15 104.25) (width 0.3) (layer "F.Cu") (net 4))
 (segment (start 156.15 104.75) (end 152.8 104.75) (width 0.3) (layer "F.Cu") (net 3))
 (segment (start 152.8 105.25) (end 156.15 105.25) (width 0.3) (layer "F.Cu") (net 2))
 (segment (start 156.15 105.75) (end 152.8 105.75) (width 0.3) (layer "F.Cu") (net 1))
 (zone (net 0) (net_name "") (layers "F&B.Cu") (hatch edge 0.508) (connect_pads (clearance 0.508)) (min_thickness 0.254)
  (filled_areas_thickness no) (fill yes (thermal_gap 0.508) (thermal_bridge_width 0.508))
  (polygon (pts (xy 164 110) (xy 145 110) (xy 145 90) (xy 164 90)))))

